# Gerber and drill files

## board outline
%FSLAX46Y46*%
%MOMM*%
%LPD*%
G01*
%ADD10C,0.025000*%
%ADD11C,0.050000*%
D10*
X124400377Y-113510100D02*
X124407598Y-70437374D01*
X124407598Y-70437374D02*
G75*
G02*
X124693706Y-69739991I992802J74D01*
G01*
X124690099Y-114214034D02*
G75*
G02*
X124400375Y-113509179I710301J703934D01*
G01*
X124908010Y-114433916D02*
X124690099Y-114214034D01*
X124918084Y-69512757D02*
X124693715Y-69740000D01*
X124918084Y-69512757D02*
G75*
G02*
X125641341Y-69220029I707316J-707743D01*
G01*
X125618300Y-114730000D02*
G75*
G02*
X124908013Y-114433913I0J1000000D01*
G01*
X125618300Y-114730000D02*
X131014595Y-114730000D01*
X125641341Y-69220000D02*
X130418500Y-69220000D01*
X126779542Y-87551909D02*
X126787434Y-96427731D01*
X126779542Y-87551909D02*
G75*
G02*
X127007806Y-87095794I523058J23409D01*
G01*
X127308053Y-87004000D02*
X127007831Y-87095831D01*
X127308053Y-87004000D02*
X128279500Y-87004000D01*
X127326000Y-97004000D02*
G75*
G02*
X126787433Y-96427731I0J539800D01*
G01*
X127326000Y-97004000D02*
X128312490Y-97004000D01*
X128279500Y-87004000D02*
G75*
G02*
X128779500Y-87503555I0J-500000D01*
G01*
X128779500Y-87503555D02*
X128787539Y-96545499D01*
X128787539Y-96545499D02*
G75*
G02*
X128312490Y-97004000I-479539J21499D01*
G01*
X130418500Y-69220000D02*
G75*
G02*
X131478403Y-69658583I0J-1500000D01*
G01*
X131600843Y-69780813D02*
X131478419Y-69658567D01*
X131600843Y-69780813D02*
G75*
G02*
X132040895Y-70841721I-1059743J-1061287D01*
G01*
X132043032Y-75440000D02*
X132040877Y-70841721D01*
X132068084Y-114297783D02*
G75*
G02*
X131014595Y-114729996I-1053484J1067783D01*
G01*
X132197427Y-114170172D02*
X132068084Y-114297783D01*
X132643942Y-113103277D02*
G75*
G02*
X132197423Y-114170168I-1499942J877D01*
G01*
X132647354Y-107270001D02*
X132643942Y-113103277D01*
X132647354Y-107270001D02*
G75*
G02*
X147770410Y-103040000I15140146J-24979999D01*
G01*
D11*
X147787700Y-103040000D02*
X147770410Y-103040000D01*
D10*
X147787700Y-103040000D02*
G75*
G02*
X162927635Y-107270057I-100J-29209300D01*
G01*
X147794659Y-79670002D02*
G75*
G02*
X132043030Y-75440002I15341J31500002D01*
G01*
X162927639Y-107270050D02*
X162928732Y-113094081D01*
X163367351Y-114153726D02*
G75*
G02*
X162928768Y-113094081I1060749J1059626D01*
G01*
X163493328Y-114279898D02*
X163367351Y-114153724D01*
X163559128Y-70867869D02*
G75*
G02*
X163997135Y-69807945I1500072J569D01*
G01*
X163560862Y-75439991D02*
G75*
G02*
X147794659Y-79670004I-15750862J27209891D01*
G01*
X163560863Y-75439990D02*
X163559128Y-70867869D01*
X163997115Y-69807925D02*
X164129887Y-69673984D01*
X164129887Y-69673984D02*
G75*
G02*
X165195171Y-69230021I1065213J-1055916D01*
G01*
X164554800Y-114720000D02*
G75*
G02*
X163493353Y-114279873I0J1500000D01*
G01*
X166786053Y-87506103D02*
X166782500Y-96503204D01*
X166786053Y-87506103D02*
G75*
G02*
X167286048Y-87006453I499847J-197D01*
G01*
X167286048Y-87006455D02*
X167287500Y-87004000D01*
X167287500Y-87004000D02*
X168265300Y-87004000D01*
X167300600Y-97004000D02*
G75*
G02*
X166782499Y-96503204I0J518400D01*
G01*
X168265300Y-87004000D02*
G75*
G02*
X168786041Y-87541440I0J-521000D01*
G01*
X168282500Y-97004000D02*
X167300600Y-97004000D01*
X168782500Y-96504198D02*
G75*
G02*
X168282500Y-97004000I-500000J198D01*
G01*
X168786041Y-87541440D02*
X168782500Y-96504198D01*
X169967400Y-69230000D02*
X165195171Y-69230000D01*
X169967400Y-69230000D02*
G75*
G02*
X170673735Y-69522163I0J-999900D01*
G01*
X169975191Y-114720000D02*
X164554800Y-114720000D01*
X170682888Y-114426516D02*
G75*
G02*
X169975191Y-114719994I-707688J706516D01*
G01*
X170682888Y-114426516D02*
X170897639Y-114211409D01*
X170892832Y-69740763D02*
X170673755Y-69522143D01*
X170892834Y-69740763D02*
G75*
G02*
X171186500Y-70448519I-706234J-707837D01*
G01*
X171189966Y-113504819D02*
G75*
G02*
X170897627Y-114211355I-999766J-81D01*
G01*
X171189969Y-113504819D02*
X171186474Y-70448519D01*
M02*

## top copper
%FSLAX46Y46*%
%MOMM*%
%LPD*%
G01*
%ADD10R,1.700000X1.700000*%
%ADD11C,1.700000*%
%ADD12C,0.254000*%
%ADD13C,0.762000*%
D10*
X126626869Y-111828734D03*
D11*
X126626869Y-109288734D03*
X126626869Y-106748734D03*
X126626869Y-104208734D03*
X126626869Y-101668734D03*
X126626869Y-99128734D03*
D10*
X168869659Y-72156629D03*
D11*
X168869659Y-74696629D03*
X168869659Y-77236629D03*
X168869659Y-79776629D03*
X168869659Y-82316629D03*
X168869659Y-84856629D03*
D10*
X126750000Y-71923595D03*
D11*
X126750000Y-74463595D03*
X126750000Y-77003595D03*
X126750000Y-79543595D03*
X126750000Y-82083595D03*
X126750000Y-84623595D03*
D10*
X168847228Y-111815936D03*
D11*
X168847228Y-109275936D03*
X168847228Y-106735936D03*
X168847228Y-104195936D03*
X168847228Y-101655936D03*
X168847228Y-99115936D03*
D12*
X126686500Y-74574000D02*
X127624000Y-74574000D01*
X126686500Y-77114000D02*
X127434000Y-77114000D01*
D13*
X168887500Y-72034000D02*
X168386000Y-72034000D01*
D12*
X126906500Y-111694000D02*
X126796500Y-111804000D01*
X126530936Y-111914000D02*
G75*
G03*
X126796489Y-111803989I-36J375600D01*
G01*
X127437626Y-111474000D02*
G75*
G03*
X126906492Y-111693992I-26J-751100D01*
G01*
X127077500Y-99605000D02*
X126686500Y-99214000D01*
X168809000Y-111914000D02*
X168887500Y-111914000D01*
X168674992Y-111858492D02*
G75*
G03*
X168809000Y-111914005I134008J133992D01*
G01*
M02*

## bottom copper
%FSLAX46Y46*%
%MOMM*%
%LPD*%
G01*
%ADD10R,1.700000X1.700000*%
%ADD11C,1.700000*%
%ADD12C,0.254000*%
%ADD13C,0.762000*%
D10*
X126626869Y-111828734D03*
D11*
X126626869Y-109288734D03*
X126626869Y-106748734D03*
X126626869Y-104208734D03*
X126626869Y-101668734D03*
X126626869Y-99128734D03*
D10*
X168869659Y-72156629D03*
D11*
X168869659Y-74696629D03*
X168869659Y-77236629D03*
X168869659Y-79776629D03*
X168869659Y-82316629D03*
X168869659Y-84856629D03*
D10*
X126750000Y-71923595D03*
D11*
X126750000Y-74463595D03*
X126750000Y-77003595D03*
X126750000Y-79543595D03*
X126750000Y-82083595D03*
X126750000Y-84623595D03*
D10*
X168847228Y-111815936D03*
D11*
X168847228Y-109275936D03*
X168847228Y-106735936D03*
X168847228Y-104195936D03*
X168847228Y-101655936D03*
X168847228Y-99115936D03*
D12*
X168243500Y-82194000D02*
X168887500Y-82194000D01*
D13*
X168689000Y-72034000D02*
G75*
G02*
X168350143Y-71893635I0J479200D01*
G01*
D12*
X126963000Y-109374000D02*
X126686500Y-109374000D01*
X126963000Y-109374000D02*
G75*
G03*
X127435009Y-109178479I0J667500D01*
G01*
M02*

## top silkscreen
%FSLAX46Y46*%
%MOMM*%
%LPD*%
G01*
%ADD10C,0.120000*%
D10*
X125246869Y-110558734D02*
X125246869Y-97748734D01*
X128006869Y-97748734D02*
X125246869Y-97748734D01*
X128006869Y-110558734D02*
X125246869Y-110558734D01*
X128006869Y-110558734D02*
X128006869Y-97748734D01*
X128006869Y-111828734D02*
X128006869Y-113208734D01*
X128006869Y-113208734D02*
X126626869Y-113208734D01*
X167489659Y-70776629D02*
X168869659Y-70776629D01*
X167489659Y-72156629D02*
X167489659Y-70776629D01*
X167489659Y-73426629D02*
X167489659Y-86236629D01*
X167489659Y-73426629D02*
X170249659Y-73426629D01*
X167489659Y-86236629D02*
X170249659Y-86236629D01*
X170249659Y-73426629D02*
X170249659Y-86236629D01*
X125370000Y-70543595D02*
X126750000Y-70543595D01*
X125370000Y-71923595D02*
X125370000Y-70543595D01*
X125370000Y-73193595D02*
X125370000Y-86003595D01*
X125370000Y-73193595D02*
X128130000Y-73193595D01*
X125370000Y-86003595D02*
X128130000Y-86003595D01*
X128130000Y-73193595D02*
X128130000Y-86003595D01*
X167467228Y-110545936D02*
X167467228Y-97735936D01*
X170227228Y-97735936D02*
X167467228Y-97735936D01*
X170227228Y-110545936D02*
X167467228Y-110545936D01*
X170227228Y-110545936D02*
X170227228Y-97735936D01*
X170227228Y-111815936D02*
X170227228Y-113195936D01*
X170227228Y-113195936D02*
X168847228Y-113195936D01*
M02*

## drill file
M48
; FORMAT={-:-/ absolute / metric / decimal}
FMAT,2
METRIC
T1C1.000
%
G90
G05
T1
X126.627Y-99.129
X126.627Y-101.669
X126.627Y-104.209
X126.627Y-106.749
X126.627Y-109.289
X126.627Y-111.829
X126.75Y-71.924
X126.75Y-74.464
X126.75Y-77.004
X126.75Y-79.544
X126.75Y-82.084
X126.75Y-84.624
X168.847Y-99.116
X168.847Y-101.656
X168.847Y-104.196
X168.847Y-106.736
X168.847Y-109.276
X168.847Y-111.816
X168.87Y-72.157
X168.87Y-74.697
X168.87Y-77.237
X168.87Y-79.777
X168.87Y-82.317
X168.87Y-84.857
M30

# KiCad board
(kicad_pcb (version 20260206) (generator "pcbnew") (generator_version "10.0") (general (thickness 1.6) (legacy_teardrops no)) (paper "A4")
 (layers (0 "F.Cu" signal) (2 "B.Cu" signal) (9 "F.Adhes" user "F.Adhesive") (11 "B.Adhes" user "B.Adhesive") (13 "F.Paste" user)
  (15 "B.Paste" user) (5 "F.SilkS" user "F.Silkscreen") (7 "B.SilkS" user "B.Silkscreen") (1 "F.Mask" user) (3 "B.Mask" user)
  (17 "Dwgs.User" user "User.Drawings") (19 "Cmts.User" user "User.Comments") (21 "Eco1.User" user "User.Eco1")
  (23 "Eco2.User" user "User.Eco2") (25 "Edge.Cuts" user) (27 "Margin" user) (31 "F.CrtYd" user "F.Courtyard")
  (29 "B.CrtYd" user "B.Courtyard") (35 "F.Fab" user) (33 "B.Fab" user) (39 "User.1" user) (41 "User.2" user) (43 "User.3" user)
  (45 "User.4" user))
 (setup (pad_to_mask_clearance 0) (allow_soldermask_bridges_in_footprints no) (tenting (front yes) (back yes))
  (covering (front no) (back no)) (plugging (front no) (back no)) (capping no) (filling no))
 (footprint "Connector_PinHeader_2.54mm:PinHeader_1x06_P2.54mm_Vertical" (layer "F.Cu") (at 126.626869 111.828734 180)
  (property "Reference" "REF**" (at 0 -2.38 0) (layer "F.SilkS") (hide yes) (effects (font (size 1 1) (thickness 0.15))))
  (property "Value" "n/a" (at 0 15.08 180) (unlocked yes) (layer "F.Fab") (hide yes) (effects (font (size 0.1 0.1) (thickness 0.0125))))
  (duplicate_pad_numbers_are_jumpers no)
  (fp_line (start 1.38 1.27) (end 1.38 14.08) (stroke (width 0.12) (type solid)) (layer "F.SilkS"))
  (fp_line (start -1.38 14.08) (end 1.38 14.08) (stroke (width 0.12) (type solid)) (layer "F.SilkS"))
  (fp_line (start -1.38 1.27) (end 1.38 1.27) (stroke (width 0.12) (type solid)) (layer "F.SilkS"))
  (fp_line (start -1.38 1.27) (end -1.38 14.08) (stroke (width 0.12) (type solid)) (layer "F.SilkS"))
  (fp_line (start -1.38 0) (end -1.38 -1.38) (stroke (width 0.12) (type solid)) (layer "F.SilkS"))
  (fp_line (start -1.38 -1.38) (end 0 -1.38) (stroke (width 0.12) (type solid)) (layer "F.SilkS"))
  (pad "1" thru_hole rect (at 0 0 180) (size 1.7 1.7) (drill 1) (layers "*.Cu" "*.Mask") (remove_unused_layers no))
  (pad "2" thru_hole circle (at 0 2.54 180) (size 1.7 1.7) (drill 1) (layers "*.Cu" "*.Mask") (remove_unused_layers no))
  (pad "3" thru_hole circle (at 0 5.08 180) (size 1.7 1.7) (drill 1) (layers "*.Cu" "*.Mask") (remove_unused_layers no))
  (pad "4" thru_hole circle (at 0 7.62 180) (size 1.7 1.7) (drill 1) (layers "*.Cu" "*.Mask") (remove_unused_layers no))
  (pad "5" thru_hole circle (at 0 10.16 180) (size 1.7 1.7) (drill 1) (layers "*.Cu" "*.Mask") (remove_unused_layers no))
  (pad "6" thru_hole circle (at 0 12.7 180) (size 1.7 1.7) (drill 1) (layers "*.Cu" "*.Mask") (remove_unused_layers no)))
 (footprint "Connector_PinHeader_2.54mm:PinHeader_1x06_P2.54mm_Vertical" (layer "F.Cu") (at 168.869659 72.156629)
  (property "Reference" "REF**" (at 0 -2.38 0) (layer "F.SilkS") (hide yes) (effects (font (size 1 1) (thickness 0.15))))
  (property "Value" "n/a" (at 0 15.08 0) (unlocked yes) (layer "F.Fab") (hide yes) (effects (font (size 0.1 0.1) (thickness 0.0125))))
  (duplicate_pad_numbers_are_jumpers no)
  (fp_line (start -1.38 -1.38) (end 0 -1.38) (stroke (width 0.12) (type solid)) (layer "F.SilkS"))
  (fp_line (start -1.38 0) (end -1.38 -1.38) (stroke (width 0.12) (type solid)) (layer "F.SilkS"))
  (fp_line (start -1.38 1.27) (end -1.38 14.08) (stroke (width 0.12) (type solid)) (layer "F.SilkS"))
  (fp_line (start -1.38 1.27) (end 1.38 1.27) (stroke (width 0.12) (type solid)) (layer "F.SilkS"))
  (fp_line (start -1.38 14.08) (end 1.38 14.08) (stroke (width 0.12) (type solid)) (layer "F.SilkS"))
  (fp_line (start 1.38 1.27) (end 1.38 14.08) (stroke (width 0.12) (type solid)) (layer "F.SilkS"))
  (pad "1" thru_hole rect (at 0 0) (size 1.7 1.7) (drill 1) (layers "*.Cu" "*.Mask") (remove_unused_layers no))
  (pad "2" thru_hole circle (at 0 2.54) (size 1.7 1.7) (drill 1) (layers "*.Cu" "*.Mask") (remove_unused_layers no))
  (pad "3" thru_hole circle (at 0 5.08) (size 1.7 1.7) (drill 1) (layers "*.Cu" "*.Mask") (remove_unused_layers no))
  (pad "4" thru_hole circle (at 0 7.62) (size 1.7 1.7) (drill 1) (layers "*.Cu" "*.Mask") (remove_unused_layers no))
  (pad "5" thru_hole circle (at 0 10.16) (size 1.7 1.7) (drill 1) (layers "*.Cu" "*.Mask") (remove_unused_layers no))
  (pad "6" thru_hole circle (at 0 12.7) (size 1.7 1.7) (drill 1) (layers "*.Cu" "*.Mask") (remove_unused_layers no)))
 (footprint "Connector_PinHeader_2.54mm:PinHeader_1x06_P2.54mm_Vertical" (layer "F.Cu") (at 126.75 71.923595)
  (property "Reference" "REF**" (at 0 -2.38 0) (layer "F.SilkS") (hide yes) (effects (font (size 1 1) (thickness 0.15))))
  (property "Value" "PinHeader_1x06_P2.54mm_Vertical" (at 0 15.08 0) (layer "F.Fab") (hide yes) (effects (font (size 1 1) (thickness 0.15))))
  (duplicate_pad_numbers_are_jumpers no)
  (fp_line (start -1.38 -1.38) (end 0 -1.38) (stroke (width 0.12) (type solid)) (layer "F.SilkS"))
  (fp_line (start -1.38 0) (end -1.38 -1.38) (stroke (width 0.12) (type solid)) (layer "F.SilkS"))
  (fp_line (start -1.38 1.27) (end -1.38 14.08) (stroke (width 0.12) (type solid)) (layer "F.SilkS"))
  (fp_line (start -1.38 1.27) (end 1.38 1.27) (stroke (width 0.12) (type solid)) (layer "F.SilkS"))
  (fp_line (start -1.38 14.08) (end 1.38 14.08) (stroke (width 0.12) (type solid)) (layer "F.SilkS"))
  (fp_line (start 1.38 1.27) (end 1.38 14.08) (stroke (width 0.12) (type solid)) (layer "F.SilkS"))
  (pad "1" thru_hole rect (at 0 0) (size 1.7 1.7) (drill 1) (layers "*.Cu" "*.Mask") (remove_unused_layers no))
  (pad "2" thru_hole circle (at 0 2.54) (size 1.7 1.7) (drill 1) (layers "*.Cu" "*.Mask") (remove_unused_layers no))
  (pad "3" thru_hole circle (at 0 5.08) (size 1.7 1.7) (drill 1) (layers "*.Cu" "*.Mask") (remove_unused_layers no))
  (pad "4" thru_hole circle (at 0 7.62) (size 1.7 1.7) (drill 1) (layers "*.Cu" "*.Mask") (remove_unused_layers no))
  (pad "5" thru_hole circle (at 0 10.16) (size 1.7 1.7) (drill 1) (layers "*.Cu" "*.Mask") (remove_unused_layers no))
  (pad "6" thru_hole circle (at 0 12.7) (size 1.7 1.7) (drill 1) (layers "*.Cu" "*.Mask") (remove_unused_layers no)))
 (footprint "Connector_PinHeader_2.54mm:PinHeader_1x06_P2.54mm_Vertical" (layer "F.Cu") (at 168.847228 111.815936 180)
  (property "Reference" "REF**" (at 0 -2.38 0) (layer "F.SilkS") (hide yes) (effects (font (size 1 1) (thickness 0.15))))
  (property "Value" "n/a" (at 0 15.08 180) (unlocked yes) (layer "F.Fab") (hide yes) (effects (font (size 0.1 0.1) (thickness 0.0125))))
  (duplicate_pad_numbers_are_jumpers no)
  (fp_line (start 1.38 1.27) (end 1.38 14.08) (stroke (width 0.12) (type solid)) (layer "F.SilkS"))
  (fp_line (start -1.38 14.08) (end 1.38 14.08) (stroke (width 0.12) (type solid)) (layer "F.SilkS"))
  (fp_line (start -1.38 1.27) (end 1.38 1.27) (stroke (width 0.12) (type solid)) (layer "F.SilkS"))
  (fp_line (start -1.38 1.27) (end -1.38 14.08) (stroke (width 0.12) (type solid)) (layer "F.SilkS"))
  (fp_line (start -1.38 0) (end -1.38 -1.38) (stroke (width 0.12) (type solid)) (layer "F.SilkS"))
  (fp_line (start -1.38 -1.38) (end 0 -1.38) (stroke (width 0.12) (type solid)) (layer "F.SilkS"))
  (pad "1" thru_hole rect (at 0 0 180) (size 1.7 1.7) (drill 1) (layers "*.Cu" "*.Mask") (remove_unused_layers no))
  (pad "2" thru_hole circle (at 0 2.54 180) (size 1.7 1.7) (drill 1) (layers "*.Cu" "*.Mask") (remove_unused_layers no))
  (pad "3" thru_hole circle (at 0 5.08 180) (size 1.7 1.7) (drill 1) (layers "*.Cu" "*.Mask") (remove_unused_layers no))
  (pad "4" thru_hole circle (at 0 7.62 180) (size 1.7 1.7) (drill 1) (layers "*.Cu" "*.Mask") (remove_unused_layers no))
  (pad "5" thru_hole circle (at 0 10.16 180) (size 1.7 1.7) (drill 1) (layers "*.Cu" "*.Mask") (remove_unused_layers no))
  (pad "6" thru_hole circle (at 0 12.7 180) (size 1.7 1.7) (drill 1) (layers "*.Cu" "*.Mask") (remove_unused_layers no)))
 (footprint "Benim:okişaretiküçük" (layer "B.Cu") (at 147.75 83.25 135)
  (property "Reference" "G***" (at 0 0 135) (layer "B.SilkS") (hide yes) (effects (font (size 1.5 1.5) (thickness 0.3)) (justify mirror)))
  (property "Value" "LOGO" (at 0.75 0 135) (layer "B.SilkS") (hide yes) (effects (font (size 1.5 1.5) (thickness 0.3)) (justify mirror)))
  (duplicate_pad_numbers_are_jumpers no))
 (gr_line (start 124.400377 113.5101) (end 124.407598 70.437374) (stroke (width 0.025) (type solid)) (layer "Edge.Cuts"))
 (gr_arc (start 124.407598 70.437374) (mid 124.481894 70.060475) (end 124.693715 69.74) (stroke (width 0.025) (type default))
  (layer "Edge.Cuts"))
 (gr_arc (start 124.690099 114.214034) (mid 124.475465 113.890292) (end 124.400377 113.509179) (stroke (width 0.025) (type default))
  (layer "Edge.Cuts"))
 (gr_line (start 124.90801 114.433916) (end 124.690099 114.214034) (stroke (width 0.025) (type solid)) (layer "Edge.Cuts"))
 (gr_line (start 124.918084 69.512757) (end 124.693715 69.74) (stroke (width 0.025) (type solid)) (layer "Edge.Cuts"))
 (gr_arc (start 124.918084 69.512757) (mid 125.242506 69.296048) (end 125.641341 69.22) (stroke (width 0.025) (type default))
  (layer "Edge.Cuts"))
 (gr_arc (start 125.6183 114.73) (mid 125.233531 114.653016) (end 124.90801 114.433916) (stroke (width 0.025) (type default))
  (layer "Edge.Cuts"))
 (gr_line (start 125.6183 114.73) (end 131.014595 114.73) (stroke (width 0.025) (type solid)) (layer "Edge.Cuts"))
 (gr_line (start 125.641341 69.22) (end 130.4185 69.22) (stroke (width 0.025) (type solid)) (layer "Edge.Cuts"))
 (gr_line (start 126.779542 87.551909) (end 126.787434 96.427731) (stroke (width 0.025) (type default)) (layer "Edge.Cuts"))
 (gr_arc (start 126.779542 87.551909) (mid 126.940006 87.150841) (end 127.007831 87.095831) (stroke (width 0.025) (type default))
  (layer "Edge.Cuts"))
 (gr_line (start 127.308053 87.004) (end 127.007831 87.095831) (stroke (width 0.025) (type default)) (layer "Edge.Cuts"))
 (gr_line (start 127.308053 87.004) (end 128.2795 87.004) (stroke (width 0.025) (type default)) (layer "Edge.Cuts"))
 (gr_arc (start 127.326 97.004) (mid 126.958691 96.859782) (end 126.787434 96.427731) (stroke (width 0.025) (type default))
  (layer "Edge.Cuts"))
 (gr_line (start 127.326 97.004) (end 128.31249 97.004) (stroke (width 0.025) (type solid)) (layer "Edge.Cuts"))
 (gr_arc (start 128.2795 87.004) (mid 128.633053 87.150447) (end 128.7795 87.503555) (stroke (width 0.025) (type default))
  (layer "Edge.Cuts"))
 (gr_line (start 128.7795 87.503555) (end 128.787539 96.545499) (stroke (width 0.025) (type default)) (layer "Edge.Cuts"))
 (gr_arc (start 128.787539 96.545499) (mid 128.655295 96.855375) (end 128.31249 97.004) (stroke (width 0.025) (type default))
  (layer "Edge.Cuts"))
 (gr_arc (start 130.4185 69.22) (mid 130.992052 69.333972) (end 131.478419 69.658567) (stroke (width 0.025) (type solid))
  (layer "Edge.Cuts"))
 (gr_line (start 131.600843 69.780813) (end 131.478419 69.658567) (stroke (width 0.025) (type solid)) (layer "Edge.Cuts"))
 (gr_arc (start 131.600843 69.780813) (mid 131.926408 70.267404) (end 132.040877 70.841721) (stroke (width 0.025) (type solid))
  (layer "Edge.Cuts"))
 (gr_line (start 132.043032 75.44) (end 132.040877 70.841721) (stroke (width 0.025) (type solid)) (layer "Edge.Cuts"))
 (gr_arc (start 132.068084 114.297783) (mid 131.583946 114.617744) (end 131.014595 114.73) (stroke (width 0.025) (type solid))
  (layer "Edge.Cuts"))
 (gr_line (start 132.197427 114.170172) (end 132.068084 114.297783) (stroke (width 0.025) (type solid)) (layer "Edge.Cuts"))
 (gr_arc (start 132.643942 113.103277) (mid 132.52765 113.681484) (end 132.197427 114.170172) (stroke (width 0.025) (type solid))
  (layer "Edge.Cuts"))
 (gr_line (start 132.647354 107.270001) (end 132.643942 113.103277) (stroke (width 0.025) (type solid)) (layer "Edge.Cuts"))
 (gr_arc (start 132.647354 107.270001) (mid 139.9215 104.119049) (end 147.77041 103.04) (stroke (width 0.025) (type solid))
  (layer "Edge.Cuts"))
 (gr_line (start 147.7877 103.04) (end 147.77041 103.04) (stroke (width 0.05) (type default)) (layer "Edge.Cuts"))
 (gr_arc (start 147.7877 103.04) (mid 156.083568 104.242867) (end 162.927639 107.27005) (stroke (width 0.025) (type solid))
  (layer "Edge.Cuts"))
 (gr_arc (start 147.794659 79.670002) (mid 139.640327 78.592143) (end 132.04303 75.440003) (stroke (width 0.025) (type solid))
  (layer "Edge.Cuts"))
 (gr_line (start 162.927639 107.27005) (end 162.928732 113.094081) (stroke (width 0.025) (type solid)) (layer "Edge.Cuts"))
 (gr_arc (start 163.367351 114.153726) (mid 163.042752 113.667489) (end 162.928784 113.094081) (stroke (width 0.025) (type solid))
  (layer "Edge.Cuts"))
 (gr_line (start 163.493328 114.279898) (end 163.367351 114.153724) (stroke (width 0.025) (type solid)) (layer "Edge.Cuts"))
 (gr_arc (start 163.559128 70.867869) (mid 163.671947 70.296514) (end 163.997115 69.807925) (stroke (width 0.025) (type solid))
  (layer "Edge.Cuts"))
 (gr_arc (start 163.560862 75.439991) (mid 155.95708 78.596083) (end 147.794659 79.670004) (stroke (width 0.025) (type solid))
  (layer "Edge.Cuts"))
 (gr_line (start 163.560863 75.43999) (end 163.559128 70.867869) (stroke (width 0.025) (type solid)) (layer "Edge.Cuts"))
 (gr_line (start 163.997115 69.807925) (end 164.129887 69.673984) (stroke (width 0.025) (type solid)) (layer "Edge.Cuts"))
 (gr_arc (start 164.129887 69.673984) (mid 164.618112 69.345431) (end 165.195171 69.23) (stroke (width 0.025) (type solid))
  (layer "Edge.Cuts"))
 (gr_arc (start 164.5548 114.72) (mid 163.980227 114.605613) (end 163.493328 114.279898) (stroke (width 0.025) (type solid))
  (layer "Edge.Cuts"))
 (gr_line (start 166.786053 87.506103) (end 166.7825 96.503204) (stroke (width 0.025) (type default)) (layer "Edge.Cuts"))
 (gr_arc (start 166.786053 87.506103) (mid 166.932457 87.152853) (end 167.286048 87.006455) (stroke (width 0.025) (type default))
  (layer "Edge.Cuts"))
 (gr_line (start 167.286048 87.006455) (end 167.2875 87.004) (stroke (width 0.025) (type default)) (layer "Edge.Cuts"))
 (gr_line (start 167.2875 87.004) (end 168.2653 87.004) (stroke (width 0.025) (type default)) (layer "Edge.Cuts"))
 (gr_arc (start 167.3006 97.004) (mid 166.941479 96.859467) (end 166.7825 96.503204) (stroke (width 0.025) (type default))
  (layer "Edge.Cuts"))
 (gr_arc (start 168.2653 87.004) (mid 168.627679 87.150667) (end 168.786041 87.54144) (stroke (width 0.025) (type default))
  (layer "Edge.Cuts"))
 (gr_line (start 168.2825 97.004) (end 167.3006 97.004) (stroke (width 0.025) (type default)) (layer "Edge.Cuts"))
 (gr_arc (start 168.7825 96.504198) (mid 168.636053 96.857553) (end 168.2825 97.004) (stroke (width 0.025) (type default))
  (layer "Edge.Cuts"))
 (gr_line (start 168.786041 87.54144) (end 168.7825 96.504198) (stroke (width 0.025) (type default)) (layer "Edge.Cuts"))
 (gr_line (start 169.9674 69.23) (end 165.195171 69.23) (stroke (width 0.025) (type solid)) (layer "Edge.Cuts"))
 (gr_arc (start 169.9674 69.23) (mid 170.349644 69.305928) (end 170.673755 69.522143) (stroke (width 0.025) (type default))
  (layer "Edge.Cuts"))
 (gr_line (start 169.975191 114.72) (end 164.5548 114.72) (stroke (width 0.025) (type solid)) (layer "Edge.Cuts"))
 (gr_arc (start 170.682888 114.426516) (mid 170.358258 114.643717) (end 169.975191 114.72) (stroke (width 0.025) (type solid))
  (layer "Edge.Cuts"))
 (gr_line (start 170.682888 114.426516) (end 170.897639 114.211409) (stroke (width 0.025) (type solid)) (layer "Edge.Cuts"))
 (gr_line (start 170.892832 69.740763) (end 170.673755 69.522143) (stroke (width 0.025) (type solid)) (layer "Edge.Cuts"))
 (gr_arc (start 170.892834 69.740763) (mid 171.110147 70.065419) (end 171.18647 70.448519) (stroke (width 0.025) (type default))
  (layer "Edge.Cuts"))
 (gr_arc (start 171.189966 113.504819) (mid 171.11402 113.887129) (end 170.897639 114.211367) (stroke (width 0.025) (type default))
  (layer "Edge.Cuts"))
 (gr_line (start 171.189969 113.504819) (end 171.186474 70.448519) (stroke (width 0.025) (type solid)) (layer "Edge.Cuts"))
 (segment (start 126.6865 74.574) (end 127.624 74.574) (width 0.254) (layer "F.Cu") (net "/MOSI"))
 (segment (start 168.2435 82.194) (end 168.8875 82.194) (width 0.254) (layer "B.Cu") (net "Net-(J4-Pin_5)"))
 (segment (start 126.6865 77.114) (end 127.434 77.114) (width 0.254) (layer "F.Cu") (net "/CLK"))
 (segment (start 168.8875 72.034) (end 168.386 72.034) (width 0.762) (layer "F.Cu") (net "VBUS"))
 (arc (start 168.689 72.034) (mid 168.505609 71.997521) (end 168.350139 71.893639) (width 0.762) (layer "B.Cu") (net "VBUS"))
 (segment (start 126.9065 111.694) (end 126.7965 111.804) (width 0.254) (layer "F.Cu") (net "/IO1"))
 (arc (start 126.530936 111.914) (mid 126.674658 111.885411) (end 126.7965 111.804) (width 0.254) (layer "F.Cu") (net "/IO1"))
 (arc (start 127.437626 111.474) (mid 127.150182 111.531176) (end 126.9065 111.694) (width 0.254) (layer "F.Cu") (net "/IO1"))
 (segment (start 127.0775 99.605) (end 126.6865 99.214) (width 0.254) (layer "F.Cu") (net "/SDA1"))
 (segment (start 168.809 111.914) (end 168.8875 111.914) (width 0.254) (layer "F.Cu") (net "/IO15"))
 (arc (start 168.674992 111.858492) (mid 168.736475 111.899573) (end 168.809 111.914) (width 0.254) (layer "F.Cu") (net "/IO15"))
 (segment (start 126.963 109.374) (end 126.6865 109.374) (width 0.254) (layer "B.Cu") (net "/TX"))
 (arc (start 126.963 109.374) (mid 127.218452 109.323187) (end 127.435014 109.178484) (width 0.254) (layer "B.Cu") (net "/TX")))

